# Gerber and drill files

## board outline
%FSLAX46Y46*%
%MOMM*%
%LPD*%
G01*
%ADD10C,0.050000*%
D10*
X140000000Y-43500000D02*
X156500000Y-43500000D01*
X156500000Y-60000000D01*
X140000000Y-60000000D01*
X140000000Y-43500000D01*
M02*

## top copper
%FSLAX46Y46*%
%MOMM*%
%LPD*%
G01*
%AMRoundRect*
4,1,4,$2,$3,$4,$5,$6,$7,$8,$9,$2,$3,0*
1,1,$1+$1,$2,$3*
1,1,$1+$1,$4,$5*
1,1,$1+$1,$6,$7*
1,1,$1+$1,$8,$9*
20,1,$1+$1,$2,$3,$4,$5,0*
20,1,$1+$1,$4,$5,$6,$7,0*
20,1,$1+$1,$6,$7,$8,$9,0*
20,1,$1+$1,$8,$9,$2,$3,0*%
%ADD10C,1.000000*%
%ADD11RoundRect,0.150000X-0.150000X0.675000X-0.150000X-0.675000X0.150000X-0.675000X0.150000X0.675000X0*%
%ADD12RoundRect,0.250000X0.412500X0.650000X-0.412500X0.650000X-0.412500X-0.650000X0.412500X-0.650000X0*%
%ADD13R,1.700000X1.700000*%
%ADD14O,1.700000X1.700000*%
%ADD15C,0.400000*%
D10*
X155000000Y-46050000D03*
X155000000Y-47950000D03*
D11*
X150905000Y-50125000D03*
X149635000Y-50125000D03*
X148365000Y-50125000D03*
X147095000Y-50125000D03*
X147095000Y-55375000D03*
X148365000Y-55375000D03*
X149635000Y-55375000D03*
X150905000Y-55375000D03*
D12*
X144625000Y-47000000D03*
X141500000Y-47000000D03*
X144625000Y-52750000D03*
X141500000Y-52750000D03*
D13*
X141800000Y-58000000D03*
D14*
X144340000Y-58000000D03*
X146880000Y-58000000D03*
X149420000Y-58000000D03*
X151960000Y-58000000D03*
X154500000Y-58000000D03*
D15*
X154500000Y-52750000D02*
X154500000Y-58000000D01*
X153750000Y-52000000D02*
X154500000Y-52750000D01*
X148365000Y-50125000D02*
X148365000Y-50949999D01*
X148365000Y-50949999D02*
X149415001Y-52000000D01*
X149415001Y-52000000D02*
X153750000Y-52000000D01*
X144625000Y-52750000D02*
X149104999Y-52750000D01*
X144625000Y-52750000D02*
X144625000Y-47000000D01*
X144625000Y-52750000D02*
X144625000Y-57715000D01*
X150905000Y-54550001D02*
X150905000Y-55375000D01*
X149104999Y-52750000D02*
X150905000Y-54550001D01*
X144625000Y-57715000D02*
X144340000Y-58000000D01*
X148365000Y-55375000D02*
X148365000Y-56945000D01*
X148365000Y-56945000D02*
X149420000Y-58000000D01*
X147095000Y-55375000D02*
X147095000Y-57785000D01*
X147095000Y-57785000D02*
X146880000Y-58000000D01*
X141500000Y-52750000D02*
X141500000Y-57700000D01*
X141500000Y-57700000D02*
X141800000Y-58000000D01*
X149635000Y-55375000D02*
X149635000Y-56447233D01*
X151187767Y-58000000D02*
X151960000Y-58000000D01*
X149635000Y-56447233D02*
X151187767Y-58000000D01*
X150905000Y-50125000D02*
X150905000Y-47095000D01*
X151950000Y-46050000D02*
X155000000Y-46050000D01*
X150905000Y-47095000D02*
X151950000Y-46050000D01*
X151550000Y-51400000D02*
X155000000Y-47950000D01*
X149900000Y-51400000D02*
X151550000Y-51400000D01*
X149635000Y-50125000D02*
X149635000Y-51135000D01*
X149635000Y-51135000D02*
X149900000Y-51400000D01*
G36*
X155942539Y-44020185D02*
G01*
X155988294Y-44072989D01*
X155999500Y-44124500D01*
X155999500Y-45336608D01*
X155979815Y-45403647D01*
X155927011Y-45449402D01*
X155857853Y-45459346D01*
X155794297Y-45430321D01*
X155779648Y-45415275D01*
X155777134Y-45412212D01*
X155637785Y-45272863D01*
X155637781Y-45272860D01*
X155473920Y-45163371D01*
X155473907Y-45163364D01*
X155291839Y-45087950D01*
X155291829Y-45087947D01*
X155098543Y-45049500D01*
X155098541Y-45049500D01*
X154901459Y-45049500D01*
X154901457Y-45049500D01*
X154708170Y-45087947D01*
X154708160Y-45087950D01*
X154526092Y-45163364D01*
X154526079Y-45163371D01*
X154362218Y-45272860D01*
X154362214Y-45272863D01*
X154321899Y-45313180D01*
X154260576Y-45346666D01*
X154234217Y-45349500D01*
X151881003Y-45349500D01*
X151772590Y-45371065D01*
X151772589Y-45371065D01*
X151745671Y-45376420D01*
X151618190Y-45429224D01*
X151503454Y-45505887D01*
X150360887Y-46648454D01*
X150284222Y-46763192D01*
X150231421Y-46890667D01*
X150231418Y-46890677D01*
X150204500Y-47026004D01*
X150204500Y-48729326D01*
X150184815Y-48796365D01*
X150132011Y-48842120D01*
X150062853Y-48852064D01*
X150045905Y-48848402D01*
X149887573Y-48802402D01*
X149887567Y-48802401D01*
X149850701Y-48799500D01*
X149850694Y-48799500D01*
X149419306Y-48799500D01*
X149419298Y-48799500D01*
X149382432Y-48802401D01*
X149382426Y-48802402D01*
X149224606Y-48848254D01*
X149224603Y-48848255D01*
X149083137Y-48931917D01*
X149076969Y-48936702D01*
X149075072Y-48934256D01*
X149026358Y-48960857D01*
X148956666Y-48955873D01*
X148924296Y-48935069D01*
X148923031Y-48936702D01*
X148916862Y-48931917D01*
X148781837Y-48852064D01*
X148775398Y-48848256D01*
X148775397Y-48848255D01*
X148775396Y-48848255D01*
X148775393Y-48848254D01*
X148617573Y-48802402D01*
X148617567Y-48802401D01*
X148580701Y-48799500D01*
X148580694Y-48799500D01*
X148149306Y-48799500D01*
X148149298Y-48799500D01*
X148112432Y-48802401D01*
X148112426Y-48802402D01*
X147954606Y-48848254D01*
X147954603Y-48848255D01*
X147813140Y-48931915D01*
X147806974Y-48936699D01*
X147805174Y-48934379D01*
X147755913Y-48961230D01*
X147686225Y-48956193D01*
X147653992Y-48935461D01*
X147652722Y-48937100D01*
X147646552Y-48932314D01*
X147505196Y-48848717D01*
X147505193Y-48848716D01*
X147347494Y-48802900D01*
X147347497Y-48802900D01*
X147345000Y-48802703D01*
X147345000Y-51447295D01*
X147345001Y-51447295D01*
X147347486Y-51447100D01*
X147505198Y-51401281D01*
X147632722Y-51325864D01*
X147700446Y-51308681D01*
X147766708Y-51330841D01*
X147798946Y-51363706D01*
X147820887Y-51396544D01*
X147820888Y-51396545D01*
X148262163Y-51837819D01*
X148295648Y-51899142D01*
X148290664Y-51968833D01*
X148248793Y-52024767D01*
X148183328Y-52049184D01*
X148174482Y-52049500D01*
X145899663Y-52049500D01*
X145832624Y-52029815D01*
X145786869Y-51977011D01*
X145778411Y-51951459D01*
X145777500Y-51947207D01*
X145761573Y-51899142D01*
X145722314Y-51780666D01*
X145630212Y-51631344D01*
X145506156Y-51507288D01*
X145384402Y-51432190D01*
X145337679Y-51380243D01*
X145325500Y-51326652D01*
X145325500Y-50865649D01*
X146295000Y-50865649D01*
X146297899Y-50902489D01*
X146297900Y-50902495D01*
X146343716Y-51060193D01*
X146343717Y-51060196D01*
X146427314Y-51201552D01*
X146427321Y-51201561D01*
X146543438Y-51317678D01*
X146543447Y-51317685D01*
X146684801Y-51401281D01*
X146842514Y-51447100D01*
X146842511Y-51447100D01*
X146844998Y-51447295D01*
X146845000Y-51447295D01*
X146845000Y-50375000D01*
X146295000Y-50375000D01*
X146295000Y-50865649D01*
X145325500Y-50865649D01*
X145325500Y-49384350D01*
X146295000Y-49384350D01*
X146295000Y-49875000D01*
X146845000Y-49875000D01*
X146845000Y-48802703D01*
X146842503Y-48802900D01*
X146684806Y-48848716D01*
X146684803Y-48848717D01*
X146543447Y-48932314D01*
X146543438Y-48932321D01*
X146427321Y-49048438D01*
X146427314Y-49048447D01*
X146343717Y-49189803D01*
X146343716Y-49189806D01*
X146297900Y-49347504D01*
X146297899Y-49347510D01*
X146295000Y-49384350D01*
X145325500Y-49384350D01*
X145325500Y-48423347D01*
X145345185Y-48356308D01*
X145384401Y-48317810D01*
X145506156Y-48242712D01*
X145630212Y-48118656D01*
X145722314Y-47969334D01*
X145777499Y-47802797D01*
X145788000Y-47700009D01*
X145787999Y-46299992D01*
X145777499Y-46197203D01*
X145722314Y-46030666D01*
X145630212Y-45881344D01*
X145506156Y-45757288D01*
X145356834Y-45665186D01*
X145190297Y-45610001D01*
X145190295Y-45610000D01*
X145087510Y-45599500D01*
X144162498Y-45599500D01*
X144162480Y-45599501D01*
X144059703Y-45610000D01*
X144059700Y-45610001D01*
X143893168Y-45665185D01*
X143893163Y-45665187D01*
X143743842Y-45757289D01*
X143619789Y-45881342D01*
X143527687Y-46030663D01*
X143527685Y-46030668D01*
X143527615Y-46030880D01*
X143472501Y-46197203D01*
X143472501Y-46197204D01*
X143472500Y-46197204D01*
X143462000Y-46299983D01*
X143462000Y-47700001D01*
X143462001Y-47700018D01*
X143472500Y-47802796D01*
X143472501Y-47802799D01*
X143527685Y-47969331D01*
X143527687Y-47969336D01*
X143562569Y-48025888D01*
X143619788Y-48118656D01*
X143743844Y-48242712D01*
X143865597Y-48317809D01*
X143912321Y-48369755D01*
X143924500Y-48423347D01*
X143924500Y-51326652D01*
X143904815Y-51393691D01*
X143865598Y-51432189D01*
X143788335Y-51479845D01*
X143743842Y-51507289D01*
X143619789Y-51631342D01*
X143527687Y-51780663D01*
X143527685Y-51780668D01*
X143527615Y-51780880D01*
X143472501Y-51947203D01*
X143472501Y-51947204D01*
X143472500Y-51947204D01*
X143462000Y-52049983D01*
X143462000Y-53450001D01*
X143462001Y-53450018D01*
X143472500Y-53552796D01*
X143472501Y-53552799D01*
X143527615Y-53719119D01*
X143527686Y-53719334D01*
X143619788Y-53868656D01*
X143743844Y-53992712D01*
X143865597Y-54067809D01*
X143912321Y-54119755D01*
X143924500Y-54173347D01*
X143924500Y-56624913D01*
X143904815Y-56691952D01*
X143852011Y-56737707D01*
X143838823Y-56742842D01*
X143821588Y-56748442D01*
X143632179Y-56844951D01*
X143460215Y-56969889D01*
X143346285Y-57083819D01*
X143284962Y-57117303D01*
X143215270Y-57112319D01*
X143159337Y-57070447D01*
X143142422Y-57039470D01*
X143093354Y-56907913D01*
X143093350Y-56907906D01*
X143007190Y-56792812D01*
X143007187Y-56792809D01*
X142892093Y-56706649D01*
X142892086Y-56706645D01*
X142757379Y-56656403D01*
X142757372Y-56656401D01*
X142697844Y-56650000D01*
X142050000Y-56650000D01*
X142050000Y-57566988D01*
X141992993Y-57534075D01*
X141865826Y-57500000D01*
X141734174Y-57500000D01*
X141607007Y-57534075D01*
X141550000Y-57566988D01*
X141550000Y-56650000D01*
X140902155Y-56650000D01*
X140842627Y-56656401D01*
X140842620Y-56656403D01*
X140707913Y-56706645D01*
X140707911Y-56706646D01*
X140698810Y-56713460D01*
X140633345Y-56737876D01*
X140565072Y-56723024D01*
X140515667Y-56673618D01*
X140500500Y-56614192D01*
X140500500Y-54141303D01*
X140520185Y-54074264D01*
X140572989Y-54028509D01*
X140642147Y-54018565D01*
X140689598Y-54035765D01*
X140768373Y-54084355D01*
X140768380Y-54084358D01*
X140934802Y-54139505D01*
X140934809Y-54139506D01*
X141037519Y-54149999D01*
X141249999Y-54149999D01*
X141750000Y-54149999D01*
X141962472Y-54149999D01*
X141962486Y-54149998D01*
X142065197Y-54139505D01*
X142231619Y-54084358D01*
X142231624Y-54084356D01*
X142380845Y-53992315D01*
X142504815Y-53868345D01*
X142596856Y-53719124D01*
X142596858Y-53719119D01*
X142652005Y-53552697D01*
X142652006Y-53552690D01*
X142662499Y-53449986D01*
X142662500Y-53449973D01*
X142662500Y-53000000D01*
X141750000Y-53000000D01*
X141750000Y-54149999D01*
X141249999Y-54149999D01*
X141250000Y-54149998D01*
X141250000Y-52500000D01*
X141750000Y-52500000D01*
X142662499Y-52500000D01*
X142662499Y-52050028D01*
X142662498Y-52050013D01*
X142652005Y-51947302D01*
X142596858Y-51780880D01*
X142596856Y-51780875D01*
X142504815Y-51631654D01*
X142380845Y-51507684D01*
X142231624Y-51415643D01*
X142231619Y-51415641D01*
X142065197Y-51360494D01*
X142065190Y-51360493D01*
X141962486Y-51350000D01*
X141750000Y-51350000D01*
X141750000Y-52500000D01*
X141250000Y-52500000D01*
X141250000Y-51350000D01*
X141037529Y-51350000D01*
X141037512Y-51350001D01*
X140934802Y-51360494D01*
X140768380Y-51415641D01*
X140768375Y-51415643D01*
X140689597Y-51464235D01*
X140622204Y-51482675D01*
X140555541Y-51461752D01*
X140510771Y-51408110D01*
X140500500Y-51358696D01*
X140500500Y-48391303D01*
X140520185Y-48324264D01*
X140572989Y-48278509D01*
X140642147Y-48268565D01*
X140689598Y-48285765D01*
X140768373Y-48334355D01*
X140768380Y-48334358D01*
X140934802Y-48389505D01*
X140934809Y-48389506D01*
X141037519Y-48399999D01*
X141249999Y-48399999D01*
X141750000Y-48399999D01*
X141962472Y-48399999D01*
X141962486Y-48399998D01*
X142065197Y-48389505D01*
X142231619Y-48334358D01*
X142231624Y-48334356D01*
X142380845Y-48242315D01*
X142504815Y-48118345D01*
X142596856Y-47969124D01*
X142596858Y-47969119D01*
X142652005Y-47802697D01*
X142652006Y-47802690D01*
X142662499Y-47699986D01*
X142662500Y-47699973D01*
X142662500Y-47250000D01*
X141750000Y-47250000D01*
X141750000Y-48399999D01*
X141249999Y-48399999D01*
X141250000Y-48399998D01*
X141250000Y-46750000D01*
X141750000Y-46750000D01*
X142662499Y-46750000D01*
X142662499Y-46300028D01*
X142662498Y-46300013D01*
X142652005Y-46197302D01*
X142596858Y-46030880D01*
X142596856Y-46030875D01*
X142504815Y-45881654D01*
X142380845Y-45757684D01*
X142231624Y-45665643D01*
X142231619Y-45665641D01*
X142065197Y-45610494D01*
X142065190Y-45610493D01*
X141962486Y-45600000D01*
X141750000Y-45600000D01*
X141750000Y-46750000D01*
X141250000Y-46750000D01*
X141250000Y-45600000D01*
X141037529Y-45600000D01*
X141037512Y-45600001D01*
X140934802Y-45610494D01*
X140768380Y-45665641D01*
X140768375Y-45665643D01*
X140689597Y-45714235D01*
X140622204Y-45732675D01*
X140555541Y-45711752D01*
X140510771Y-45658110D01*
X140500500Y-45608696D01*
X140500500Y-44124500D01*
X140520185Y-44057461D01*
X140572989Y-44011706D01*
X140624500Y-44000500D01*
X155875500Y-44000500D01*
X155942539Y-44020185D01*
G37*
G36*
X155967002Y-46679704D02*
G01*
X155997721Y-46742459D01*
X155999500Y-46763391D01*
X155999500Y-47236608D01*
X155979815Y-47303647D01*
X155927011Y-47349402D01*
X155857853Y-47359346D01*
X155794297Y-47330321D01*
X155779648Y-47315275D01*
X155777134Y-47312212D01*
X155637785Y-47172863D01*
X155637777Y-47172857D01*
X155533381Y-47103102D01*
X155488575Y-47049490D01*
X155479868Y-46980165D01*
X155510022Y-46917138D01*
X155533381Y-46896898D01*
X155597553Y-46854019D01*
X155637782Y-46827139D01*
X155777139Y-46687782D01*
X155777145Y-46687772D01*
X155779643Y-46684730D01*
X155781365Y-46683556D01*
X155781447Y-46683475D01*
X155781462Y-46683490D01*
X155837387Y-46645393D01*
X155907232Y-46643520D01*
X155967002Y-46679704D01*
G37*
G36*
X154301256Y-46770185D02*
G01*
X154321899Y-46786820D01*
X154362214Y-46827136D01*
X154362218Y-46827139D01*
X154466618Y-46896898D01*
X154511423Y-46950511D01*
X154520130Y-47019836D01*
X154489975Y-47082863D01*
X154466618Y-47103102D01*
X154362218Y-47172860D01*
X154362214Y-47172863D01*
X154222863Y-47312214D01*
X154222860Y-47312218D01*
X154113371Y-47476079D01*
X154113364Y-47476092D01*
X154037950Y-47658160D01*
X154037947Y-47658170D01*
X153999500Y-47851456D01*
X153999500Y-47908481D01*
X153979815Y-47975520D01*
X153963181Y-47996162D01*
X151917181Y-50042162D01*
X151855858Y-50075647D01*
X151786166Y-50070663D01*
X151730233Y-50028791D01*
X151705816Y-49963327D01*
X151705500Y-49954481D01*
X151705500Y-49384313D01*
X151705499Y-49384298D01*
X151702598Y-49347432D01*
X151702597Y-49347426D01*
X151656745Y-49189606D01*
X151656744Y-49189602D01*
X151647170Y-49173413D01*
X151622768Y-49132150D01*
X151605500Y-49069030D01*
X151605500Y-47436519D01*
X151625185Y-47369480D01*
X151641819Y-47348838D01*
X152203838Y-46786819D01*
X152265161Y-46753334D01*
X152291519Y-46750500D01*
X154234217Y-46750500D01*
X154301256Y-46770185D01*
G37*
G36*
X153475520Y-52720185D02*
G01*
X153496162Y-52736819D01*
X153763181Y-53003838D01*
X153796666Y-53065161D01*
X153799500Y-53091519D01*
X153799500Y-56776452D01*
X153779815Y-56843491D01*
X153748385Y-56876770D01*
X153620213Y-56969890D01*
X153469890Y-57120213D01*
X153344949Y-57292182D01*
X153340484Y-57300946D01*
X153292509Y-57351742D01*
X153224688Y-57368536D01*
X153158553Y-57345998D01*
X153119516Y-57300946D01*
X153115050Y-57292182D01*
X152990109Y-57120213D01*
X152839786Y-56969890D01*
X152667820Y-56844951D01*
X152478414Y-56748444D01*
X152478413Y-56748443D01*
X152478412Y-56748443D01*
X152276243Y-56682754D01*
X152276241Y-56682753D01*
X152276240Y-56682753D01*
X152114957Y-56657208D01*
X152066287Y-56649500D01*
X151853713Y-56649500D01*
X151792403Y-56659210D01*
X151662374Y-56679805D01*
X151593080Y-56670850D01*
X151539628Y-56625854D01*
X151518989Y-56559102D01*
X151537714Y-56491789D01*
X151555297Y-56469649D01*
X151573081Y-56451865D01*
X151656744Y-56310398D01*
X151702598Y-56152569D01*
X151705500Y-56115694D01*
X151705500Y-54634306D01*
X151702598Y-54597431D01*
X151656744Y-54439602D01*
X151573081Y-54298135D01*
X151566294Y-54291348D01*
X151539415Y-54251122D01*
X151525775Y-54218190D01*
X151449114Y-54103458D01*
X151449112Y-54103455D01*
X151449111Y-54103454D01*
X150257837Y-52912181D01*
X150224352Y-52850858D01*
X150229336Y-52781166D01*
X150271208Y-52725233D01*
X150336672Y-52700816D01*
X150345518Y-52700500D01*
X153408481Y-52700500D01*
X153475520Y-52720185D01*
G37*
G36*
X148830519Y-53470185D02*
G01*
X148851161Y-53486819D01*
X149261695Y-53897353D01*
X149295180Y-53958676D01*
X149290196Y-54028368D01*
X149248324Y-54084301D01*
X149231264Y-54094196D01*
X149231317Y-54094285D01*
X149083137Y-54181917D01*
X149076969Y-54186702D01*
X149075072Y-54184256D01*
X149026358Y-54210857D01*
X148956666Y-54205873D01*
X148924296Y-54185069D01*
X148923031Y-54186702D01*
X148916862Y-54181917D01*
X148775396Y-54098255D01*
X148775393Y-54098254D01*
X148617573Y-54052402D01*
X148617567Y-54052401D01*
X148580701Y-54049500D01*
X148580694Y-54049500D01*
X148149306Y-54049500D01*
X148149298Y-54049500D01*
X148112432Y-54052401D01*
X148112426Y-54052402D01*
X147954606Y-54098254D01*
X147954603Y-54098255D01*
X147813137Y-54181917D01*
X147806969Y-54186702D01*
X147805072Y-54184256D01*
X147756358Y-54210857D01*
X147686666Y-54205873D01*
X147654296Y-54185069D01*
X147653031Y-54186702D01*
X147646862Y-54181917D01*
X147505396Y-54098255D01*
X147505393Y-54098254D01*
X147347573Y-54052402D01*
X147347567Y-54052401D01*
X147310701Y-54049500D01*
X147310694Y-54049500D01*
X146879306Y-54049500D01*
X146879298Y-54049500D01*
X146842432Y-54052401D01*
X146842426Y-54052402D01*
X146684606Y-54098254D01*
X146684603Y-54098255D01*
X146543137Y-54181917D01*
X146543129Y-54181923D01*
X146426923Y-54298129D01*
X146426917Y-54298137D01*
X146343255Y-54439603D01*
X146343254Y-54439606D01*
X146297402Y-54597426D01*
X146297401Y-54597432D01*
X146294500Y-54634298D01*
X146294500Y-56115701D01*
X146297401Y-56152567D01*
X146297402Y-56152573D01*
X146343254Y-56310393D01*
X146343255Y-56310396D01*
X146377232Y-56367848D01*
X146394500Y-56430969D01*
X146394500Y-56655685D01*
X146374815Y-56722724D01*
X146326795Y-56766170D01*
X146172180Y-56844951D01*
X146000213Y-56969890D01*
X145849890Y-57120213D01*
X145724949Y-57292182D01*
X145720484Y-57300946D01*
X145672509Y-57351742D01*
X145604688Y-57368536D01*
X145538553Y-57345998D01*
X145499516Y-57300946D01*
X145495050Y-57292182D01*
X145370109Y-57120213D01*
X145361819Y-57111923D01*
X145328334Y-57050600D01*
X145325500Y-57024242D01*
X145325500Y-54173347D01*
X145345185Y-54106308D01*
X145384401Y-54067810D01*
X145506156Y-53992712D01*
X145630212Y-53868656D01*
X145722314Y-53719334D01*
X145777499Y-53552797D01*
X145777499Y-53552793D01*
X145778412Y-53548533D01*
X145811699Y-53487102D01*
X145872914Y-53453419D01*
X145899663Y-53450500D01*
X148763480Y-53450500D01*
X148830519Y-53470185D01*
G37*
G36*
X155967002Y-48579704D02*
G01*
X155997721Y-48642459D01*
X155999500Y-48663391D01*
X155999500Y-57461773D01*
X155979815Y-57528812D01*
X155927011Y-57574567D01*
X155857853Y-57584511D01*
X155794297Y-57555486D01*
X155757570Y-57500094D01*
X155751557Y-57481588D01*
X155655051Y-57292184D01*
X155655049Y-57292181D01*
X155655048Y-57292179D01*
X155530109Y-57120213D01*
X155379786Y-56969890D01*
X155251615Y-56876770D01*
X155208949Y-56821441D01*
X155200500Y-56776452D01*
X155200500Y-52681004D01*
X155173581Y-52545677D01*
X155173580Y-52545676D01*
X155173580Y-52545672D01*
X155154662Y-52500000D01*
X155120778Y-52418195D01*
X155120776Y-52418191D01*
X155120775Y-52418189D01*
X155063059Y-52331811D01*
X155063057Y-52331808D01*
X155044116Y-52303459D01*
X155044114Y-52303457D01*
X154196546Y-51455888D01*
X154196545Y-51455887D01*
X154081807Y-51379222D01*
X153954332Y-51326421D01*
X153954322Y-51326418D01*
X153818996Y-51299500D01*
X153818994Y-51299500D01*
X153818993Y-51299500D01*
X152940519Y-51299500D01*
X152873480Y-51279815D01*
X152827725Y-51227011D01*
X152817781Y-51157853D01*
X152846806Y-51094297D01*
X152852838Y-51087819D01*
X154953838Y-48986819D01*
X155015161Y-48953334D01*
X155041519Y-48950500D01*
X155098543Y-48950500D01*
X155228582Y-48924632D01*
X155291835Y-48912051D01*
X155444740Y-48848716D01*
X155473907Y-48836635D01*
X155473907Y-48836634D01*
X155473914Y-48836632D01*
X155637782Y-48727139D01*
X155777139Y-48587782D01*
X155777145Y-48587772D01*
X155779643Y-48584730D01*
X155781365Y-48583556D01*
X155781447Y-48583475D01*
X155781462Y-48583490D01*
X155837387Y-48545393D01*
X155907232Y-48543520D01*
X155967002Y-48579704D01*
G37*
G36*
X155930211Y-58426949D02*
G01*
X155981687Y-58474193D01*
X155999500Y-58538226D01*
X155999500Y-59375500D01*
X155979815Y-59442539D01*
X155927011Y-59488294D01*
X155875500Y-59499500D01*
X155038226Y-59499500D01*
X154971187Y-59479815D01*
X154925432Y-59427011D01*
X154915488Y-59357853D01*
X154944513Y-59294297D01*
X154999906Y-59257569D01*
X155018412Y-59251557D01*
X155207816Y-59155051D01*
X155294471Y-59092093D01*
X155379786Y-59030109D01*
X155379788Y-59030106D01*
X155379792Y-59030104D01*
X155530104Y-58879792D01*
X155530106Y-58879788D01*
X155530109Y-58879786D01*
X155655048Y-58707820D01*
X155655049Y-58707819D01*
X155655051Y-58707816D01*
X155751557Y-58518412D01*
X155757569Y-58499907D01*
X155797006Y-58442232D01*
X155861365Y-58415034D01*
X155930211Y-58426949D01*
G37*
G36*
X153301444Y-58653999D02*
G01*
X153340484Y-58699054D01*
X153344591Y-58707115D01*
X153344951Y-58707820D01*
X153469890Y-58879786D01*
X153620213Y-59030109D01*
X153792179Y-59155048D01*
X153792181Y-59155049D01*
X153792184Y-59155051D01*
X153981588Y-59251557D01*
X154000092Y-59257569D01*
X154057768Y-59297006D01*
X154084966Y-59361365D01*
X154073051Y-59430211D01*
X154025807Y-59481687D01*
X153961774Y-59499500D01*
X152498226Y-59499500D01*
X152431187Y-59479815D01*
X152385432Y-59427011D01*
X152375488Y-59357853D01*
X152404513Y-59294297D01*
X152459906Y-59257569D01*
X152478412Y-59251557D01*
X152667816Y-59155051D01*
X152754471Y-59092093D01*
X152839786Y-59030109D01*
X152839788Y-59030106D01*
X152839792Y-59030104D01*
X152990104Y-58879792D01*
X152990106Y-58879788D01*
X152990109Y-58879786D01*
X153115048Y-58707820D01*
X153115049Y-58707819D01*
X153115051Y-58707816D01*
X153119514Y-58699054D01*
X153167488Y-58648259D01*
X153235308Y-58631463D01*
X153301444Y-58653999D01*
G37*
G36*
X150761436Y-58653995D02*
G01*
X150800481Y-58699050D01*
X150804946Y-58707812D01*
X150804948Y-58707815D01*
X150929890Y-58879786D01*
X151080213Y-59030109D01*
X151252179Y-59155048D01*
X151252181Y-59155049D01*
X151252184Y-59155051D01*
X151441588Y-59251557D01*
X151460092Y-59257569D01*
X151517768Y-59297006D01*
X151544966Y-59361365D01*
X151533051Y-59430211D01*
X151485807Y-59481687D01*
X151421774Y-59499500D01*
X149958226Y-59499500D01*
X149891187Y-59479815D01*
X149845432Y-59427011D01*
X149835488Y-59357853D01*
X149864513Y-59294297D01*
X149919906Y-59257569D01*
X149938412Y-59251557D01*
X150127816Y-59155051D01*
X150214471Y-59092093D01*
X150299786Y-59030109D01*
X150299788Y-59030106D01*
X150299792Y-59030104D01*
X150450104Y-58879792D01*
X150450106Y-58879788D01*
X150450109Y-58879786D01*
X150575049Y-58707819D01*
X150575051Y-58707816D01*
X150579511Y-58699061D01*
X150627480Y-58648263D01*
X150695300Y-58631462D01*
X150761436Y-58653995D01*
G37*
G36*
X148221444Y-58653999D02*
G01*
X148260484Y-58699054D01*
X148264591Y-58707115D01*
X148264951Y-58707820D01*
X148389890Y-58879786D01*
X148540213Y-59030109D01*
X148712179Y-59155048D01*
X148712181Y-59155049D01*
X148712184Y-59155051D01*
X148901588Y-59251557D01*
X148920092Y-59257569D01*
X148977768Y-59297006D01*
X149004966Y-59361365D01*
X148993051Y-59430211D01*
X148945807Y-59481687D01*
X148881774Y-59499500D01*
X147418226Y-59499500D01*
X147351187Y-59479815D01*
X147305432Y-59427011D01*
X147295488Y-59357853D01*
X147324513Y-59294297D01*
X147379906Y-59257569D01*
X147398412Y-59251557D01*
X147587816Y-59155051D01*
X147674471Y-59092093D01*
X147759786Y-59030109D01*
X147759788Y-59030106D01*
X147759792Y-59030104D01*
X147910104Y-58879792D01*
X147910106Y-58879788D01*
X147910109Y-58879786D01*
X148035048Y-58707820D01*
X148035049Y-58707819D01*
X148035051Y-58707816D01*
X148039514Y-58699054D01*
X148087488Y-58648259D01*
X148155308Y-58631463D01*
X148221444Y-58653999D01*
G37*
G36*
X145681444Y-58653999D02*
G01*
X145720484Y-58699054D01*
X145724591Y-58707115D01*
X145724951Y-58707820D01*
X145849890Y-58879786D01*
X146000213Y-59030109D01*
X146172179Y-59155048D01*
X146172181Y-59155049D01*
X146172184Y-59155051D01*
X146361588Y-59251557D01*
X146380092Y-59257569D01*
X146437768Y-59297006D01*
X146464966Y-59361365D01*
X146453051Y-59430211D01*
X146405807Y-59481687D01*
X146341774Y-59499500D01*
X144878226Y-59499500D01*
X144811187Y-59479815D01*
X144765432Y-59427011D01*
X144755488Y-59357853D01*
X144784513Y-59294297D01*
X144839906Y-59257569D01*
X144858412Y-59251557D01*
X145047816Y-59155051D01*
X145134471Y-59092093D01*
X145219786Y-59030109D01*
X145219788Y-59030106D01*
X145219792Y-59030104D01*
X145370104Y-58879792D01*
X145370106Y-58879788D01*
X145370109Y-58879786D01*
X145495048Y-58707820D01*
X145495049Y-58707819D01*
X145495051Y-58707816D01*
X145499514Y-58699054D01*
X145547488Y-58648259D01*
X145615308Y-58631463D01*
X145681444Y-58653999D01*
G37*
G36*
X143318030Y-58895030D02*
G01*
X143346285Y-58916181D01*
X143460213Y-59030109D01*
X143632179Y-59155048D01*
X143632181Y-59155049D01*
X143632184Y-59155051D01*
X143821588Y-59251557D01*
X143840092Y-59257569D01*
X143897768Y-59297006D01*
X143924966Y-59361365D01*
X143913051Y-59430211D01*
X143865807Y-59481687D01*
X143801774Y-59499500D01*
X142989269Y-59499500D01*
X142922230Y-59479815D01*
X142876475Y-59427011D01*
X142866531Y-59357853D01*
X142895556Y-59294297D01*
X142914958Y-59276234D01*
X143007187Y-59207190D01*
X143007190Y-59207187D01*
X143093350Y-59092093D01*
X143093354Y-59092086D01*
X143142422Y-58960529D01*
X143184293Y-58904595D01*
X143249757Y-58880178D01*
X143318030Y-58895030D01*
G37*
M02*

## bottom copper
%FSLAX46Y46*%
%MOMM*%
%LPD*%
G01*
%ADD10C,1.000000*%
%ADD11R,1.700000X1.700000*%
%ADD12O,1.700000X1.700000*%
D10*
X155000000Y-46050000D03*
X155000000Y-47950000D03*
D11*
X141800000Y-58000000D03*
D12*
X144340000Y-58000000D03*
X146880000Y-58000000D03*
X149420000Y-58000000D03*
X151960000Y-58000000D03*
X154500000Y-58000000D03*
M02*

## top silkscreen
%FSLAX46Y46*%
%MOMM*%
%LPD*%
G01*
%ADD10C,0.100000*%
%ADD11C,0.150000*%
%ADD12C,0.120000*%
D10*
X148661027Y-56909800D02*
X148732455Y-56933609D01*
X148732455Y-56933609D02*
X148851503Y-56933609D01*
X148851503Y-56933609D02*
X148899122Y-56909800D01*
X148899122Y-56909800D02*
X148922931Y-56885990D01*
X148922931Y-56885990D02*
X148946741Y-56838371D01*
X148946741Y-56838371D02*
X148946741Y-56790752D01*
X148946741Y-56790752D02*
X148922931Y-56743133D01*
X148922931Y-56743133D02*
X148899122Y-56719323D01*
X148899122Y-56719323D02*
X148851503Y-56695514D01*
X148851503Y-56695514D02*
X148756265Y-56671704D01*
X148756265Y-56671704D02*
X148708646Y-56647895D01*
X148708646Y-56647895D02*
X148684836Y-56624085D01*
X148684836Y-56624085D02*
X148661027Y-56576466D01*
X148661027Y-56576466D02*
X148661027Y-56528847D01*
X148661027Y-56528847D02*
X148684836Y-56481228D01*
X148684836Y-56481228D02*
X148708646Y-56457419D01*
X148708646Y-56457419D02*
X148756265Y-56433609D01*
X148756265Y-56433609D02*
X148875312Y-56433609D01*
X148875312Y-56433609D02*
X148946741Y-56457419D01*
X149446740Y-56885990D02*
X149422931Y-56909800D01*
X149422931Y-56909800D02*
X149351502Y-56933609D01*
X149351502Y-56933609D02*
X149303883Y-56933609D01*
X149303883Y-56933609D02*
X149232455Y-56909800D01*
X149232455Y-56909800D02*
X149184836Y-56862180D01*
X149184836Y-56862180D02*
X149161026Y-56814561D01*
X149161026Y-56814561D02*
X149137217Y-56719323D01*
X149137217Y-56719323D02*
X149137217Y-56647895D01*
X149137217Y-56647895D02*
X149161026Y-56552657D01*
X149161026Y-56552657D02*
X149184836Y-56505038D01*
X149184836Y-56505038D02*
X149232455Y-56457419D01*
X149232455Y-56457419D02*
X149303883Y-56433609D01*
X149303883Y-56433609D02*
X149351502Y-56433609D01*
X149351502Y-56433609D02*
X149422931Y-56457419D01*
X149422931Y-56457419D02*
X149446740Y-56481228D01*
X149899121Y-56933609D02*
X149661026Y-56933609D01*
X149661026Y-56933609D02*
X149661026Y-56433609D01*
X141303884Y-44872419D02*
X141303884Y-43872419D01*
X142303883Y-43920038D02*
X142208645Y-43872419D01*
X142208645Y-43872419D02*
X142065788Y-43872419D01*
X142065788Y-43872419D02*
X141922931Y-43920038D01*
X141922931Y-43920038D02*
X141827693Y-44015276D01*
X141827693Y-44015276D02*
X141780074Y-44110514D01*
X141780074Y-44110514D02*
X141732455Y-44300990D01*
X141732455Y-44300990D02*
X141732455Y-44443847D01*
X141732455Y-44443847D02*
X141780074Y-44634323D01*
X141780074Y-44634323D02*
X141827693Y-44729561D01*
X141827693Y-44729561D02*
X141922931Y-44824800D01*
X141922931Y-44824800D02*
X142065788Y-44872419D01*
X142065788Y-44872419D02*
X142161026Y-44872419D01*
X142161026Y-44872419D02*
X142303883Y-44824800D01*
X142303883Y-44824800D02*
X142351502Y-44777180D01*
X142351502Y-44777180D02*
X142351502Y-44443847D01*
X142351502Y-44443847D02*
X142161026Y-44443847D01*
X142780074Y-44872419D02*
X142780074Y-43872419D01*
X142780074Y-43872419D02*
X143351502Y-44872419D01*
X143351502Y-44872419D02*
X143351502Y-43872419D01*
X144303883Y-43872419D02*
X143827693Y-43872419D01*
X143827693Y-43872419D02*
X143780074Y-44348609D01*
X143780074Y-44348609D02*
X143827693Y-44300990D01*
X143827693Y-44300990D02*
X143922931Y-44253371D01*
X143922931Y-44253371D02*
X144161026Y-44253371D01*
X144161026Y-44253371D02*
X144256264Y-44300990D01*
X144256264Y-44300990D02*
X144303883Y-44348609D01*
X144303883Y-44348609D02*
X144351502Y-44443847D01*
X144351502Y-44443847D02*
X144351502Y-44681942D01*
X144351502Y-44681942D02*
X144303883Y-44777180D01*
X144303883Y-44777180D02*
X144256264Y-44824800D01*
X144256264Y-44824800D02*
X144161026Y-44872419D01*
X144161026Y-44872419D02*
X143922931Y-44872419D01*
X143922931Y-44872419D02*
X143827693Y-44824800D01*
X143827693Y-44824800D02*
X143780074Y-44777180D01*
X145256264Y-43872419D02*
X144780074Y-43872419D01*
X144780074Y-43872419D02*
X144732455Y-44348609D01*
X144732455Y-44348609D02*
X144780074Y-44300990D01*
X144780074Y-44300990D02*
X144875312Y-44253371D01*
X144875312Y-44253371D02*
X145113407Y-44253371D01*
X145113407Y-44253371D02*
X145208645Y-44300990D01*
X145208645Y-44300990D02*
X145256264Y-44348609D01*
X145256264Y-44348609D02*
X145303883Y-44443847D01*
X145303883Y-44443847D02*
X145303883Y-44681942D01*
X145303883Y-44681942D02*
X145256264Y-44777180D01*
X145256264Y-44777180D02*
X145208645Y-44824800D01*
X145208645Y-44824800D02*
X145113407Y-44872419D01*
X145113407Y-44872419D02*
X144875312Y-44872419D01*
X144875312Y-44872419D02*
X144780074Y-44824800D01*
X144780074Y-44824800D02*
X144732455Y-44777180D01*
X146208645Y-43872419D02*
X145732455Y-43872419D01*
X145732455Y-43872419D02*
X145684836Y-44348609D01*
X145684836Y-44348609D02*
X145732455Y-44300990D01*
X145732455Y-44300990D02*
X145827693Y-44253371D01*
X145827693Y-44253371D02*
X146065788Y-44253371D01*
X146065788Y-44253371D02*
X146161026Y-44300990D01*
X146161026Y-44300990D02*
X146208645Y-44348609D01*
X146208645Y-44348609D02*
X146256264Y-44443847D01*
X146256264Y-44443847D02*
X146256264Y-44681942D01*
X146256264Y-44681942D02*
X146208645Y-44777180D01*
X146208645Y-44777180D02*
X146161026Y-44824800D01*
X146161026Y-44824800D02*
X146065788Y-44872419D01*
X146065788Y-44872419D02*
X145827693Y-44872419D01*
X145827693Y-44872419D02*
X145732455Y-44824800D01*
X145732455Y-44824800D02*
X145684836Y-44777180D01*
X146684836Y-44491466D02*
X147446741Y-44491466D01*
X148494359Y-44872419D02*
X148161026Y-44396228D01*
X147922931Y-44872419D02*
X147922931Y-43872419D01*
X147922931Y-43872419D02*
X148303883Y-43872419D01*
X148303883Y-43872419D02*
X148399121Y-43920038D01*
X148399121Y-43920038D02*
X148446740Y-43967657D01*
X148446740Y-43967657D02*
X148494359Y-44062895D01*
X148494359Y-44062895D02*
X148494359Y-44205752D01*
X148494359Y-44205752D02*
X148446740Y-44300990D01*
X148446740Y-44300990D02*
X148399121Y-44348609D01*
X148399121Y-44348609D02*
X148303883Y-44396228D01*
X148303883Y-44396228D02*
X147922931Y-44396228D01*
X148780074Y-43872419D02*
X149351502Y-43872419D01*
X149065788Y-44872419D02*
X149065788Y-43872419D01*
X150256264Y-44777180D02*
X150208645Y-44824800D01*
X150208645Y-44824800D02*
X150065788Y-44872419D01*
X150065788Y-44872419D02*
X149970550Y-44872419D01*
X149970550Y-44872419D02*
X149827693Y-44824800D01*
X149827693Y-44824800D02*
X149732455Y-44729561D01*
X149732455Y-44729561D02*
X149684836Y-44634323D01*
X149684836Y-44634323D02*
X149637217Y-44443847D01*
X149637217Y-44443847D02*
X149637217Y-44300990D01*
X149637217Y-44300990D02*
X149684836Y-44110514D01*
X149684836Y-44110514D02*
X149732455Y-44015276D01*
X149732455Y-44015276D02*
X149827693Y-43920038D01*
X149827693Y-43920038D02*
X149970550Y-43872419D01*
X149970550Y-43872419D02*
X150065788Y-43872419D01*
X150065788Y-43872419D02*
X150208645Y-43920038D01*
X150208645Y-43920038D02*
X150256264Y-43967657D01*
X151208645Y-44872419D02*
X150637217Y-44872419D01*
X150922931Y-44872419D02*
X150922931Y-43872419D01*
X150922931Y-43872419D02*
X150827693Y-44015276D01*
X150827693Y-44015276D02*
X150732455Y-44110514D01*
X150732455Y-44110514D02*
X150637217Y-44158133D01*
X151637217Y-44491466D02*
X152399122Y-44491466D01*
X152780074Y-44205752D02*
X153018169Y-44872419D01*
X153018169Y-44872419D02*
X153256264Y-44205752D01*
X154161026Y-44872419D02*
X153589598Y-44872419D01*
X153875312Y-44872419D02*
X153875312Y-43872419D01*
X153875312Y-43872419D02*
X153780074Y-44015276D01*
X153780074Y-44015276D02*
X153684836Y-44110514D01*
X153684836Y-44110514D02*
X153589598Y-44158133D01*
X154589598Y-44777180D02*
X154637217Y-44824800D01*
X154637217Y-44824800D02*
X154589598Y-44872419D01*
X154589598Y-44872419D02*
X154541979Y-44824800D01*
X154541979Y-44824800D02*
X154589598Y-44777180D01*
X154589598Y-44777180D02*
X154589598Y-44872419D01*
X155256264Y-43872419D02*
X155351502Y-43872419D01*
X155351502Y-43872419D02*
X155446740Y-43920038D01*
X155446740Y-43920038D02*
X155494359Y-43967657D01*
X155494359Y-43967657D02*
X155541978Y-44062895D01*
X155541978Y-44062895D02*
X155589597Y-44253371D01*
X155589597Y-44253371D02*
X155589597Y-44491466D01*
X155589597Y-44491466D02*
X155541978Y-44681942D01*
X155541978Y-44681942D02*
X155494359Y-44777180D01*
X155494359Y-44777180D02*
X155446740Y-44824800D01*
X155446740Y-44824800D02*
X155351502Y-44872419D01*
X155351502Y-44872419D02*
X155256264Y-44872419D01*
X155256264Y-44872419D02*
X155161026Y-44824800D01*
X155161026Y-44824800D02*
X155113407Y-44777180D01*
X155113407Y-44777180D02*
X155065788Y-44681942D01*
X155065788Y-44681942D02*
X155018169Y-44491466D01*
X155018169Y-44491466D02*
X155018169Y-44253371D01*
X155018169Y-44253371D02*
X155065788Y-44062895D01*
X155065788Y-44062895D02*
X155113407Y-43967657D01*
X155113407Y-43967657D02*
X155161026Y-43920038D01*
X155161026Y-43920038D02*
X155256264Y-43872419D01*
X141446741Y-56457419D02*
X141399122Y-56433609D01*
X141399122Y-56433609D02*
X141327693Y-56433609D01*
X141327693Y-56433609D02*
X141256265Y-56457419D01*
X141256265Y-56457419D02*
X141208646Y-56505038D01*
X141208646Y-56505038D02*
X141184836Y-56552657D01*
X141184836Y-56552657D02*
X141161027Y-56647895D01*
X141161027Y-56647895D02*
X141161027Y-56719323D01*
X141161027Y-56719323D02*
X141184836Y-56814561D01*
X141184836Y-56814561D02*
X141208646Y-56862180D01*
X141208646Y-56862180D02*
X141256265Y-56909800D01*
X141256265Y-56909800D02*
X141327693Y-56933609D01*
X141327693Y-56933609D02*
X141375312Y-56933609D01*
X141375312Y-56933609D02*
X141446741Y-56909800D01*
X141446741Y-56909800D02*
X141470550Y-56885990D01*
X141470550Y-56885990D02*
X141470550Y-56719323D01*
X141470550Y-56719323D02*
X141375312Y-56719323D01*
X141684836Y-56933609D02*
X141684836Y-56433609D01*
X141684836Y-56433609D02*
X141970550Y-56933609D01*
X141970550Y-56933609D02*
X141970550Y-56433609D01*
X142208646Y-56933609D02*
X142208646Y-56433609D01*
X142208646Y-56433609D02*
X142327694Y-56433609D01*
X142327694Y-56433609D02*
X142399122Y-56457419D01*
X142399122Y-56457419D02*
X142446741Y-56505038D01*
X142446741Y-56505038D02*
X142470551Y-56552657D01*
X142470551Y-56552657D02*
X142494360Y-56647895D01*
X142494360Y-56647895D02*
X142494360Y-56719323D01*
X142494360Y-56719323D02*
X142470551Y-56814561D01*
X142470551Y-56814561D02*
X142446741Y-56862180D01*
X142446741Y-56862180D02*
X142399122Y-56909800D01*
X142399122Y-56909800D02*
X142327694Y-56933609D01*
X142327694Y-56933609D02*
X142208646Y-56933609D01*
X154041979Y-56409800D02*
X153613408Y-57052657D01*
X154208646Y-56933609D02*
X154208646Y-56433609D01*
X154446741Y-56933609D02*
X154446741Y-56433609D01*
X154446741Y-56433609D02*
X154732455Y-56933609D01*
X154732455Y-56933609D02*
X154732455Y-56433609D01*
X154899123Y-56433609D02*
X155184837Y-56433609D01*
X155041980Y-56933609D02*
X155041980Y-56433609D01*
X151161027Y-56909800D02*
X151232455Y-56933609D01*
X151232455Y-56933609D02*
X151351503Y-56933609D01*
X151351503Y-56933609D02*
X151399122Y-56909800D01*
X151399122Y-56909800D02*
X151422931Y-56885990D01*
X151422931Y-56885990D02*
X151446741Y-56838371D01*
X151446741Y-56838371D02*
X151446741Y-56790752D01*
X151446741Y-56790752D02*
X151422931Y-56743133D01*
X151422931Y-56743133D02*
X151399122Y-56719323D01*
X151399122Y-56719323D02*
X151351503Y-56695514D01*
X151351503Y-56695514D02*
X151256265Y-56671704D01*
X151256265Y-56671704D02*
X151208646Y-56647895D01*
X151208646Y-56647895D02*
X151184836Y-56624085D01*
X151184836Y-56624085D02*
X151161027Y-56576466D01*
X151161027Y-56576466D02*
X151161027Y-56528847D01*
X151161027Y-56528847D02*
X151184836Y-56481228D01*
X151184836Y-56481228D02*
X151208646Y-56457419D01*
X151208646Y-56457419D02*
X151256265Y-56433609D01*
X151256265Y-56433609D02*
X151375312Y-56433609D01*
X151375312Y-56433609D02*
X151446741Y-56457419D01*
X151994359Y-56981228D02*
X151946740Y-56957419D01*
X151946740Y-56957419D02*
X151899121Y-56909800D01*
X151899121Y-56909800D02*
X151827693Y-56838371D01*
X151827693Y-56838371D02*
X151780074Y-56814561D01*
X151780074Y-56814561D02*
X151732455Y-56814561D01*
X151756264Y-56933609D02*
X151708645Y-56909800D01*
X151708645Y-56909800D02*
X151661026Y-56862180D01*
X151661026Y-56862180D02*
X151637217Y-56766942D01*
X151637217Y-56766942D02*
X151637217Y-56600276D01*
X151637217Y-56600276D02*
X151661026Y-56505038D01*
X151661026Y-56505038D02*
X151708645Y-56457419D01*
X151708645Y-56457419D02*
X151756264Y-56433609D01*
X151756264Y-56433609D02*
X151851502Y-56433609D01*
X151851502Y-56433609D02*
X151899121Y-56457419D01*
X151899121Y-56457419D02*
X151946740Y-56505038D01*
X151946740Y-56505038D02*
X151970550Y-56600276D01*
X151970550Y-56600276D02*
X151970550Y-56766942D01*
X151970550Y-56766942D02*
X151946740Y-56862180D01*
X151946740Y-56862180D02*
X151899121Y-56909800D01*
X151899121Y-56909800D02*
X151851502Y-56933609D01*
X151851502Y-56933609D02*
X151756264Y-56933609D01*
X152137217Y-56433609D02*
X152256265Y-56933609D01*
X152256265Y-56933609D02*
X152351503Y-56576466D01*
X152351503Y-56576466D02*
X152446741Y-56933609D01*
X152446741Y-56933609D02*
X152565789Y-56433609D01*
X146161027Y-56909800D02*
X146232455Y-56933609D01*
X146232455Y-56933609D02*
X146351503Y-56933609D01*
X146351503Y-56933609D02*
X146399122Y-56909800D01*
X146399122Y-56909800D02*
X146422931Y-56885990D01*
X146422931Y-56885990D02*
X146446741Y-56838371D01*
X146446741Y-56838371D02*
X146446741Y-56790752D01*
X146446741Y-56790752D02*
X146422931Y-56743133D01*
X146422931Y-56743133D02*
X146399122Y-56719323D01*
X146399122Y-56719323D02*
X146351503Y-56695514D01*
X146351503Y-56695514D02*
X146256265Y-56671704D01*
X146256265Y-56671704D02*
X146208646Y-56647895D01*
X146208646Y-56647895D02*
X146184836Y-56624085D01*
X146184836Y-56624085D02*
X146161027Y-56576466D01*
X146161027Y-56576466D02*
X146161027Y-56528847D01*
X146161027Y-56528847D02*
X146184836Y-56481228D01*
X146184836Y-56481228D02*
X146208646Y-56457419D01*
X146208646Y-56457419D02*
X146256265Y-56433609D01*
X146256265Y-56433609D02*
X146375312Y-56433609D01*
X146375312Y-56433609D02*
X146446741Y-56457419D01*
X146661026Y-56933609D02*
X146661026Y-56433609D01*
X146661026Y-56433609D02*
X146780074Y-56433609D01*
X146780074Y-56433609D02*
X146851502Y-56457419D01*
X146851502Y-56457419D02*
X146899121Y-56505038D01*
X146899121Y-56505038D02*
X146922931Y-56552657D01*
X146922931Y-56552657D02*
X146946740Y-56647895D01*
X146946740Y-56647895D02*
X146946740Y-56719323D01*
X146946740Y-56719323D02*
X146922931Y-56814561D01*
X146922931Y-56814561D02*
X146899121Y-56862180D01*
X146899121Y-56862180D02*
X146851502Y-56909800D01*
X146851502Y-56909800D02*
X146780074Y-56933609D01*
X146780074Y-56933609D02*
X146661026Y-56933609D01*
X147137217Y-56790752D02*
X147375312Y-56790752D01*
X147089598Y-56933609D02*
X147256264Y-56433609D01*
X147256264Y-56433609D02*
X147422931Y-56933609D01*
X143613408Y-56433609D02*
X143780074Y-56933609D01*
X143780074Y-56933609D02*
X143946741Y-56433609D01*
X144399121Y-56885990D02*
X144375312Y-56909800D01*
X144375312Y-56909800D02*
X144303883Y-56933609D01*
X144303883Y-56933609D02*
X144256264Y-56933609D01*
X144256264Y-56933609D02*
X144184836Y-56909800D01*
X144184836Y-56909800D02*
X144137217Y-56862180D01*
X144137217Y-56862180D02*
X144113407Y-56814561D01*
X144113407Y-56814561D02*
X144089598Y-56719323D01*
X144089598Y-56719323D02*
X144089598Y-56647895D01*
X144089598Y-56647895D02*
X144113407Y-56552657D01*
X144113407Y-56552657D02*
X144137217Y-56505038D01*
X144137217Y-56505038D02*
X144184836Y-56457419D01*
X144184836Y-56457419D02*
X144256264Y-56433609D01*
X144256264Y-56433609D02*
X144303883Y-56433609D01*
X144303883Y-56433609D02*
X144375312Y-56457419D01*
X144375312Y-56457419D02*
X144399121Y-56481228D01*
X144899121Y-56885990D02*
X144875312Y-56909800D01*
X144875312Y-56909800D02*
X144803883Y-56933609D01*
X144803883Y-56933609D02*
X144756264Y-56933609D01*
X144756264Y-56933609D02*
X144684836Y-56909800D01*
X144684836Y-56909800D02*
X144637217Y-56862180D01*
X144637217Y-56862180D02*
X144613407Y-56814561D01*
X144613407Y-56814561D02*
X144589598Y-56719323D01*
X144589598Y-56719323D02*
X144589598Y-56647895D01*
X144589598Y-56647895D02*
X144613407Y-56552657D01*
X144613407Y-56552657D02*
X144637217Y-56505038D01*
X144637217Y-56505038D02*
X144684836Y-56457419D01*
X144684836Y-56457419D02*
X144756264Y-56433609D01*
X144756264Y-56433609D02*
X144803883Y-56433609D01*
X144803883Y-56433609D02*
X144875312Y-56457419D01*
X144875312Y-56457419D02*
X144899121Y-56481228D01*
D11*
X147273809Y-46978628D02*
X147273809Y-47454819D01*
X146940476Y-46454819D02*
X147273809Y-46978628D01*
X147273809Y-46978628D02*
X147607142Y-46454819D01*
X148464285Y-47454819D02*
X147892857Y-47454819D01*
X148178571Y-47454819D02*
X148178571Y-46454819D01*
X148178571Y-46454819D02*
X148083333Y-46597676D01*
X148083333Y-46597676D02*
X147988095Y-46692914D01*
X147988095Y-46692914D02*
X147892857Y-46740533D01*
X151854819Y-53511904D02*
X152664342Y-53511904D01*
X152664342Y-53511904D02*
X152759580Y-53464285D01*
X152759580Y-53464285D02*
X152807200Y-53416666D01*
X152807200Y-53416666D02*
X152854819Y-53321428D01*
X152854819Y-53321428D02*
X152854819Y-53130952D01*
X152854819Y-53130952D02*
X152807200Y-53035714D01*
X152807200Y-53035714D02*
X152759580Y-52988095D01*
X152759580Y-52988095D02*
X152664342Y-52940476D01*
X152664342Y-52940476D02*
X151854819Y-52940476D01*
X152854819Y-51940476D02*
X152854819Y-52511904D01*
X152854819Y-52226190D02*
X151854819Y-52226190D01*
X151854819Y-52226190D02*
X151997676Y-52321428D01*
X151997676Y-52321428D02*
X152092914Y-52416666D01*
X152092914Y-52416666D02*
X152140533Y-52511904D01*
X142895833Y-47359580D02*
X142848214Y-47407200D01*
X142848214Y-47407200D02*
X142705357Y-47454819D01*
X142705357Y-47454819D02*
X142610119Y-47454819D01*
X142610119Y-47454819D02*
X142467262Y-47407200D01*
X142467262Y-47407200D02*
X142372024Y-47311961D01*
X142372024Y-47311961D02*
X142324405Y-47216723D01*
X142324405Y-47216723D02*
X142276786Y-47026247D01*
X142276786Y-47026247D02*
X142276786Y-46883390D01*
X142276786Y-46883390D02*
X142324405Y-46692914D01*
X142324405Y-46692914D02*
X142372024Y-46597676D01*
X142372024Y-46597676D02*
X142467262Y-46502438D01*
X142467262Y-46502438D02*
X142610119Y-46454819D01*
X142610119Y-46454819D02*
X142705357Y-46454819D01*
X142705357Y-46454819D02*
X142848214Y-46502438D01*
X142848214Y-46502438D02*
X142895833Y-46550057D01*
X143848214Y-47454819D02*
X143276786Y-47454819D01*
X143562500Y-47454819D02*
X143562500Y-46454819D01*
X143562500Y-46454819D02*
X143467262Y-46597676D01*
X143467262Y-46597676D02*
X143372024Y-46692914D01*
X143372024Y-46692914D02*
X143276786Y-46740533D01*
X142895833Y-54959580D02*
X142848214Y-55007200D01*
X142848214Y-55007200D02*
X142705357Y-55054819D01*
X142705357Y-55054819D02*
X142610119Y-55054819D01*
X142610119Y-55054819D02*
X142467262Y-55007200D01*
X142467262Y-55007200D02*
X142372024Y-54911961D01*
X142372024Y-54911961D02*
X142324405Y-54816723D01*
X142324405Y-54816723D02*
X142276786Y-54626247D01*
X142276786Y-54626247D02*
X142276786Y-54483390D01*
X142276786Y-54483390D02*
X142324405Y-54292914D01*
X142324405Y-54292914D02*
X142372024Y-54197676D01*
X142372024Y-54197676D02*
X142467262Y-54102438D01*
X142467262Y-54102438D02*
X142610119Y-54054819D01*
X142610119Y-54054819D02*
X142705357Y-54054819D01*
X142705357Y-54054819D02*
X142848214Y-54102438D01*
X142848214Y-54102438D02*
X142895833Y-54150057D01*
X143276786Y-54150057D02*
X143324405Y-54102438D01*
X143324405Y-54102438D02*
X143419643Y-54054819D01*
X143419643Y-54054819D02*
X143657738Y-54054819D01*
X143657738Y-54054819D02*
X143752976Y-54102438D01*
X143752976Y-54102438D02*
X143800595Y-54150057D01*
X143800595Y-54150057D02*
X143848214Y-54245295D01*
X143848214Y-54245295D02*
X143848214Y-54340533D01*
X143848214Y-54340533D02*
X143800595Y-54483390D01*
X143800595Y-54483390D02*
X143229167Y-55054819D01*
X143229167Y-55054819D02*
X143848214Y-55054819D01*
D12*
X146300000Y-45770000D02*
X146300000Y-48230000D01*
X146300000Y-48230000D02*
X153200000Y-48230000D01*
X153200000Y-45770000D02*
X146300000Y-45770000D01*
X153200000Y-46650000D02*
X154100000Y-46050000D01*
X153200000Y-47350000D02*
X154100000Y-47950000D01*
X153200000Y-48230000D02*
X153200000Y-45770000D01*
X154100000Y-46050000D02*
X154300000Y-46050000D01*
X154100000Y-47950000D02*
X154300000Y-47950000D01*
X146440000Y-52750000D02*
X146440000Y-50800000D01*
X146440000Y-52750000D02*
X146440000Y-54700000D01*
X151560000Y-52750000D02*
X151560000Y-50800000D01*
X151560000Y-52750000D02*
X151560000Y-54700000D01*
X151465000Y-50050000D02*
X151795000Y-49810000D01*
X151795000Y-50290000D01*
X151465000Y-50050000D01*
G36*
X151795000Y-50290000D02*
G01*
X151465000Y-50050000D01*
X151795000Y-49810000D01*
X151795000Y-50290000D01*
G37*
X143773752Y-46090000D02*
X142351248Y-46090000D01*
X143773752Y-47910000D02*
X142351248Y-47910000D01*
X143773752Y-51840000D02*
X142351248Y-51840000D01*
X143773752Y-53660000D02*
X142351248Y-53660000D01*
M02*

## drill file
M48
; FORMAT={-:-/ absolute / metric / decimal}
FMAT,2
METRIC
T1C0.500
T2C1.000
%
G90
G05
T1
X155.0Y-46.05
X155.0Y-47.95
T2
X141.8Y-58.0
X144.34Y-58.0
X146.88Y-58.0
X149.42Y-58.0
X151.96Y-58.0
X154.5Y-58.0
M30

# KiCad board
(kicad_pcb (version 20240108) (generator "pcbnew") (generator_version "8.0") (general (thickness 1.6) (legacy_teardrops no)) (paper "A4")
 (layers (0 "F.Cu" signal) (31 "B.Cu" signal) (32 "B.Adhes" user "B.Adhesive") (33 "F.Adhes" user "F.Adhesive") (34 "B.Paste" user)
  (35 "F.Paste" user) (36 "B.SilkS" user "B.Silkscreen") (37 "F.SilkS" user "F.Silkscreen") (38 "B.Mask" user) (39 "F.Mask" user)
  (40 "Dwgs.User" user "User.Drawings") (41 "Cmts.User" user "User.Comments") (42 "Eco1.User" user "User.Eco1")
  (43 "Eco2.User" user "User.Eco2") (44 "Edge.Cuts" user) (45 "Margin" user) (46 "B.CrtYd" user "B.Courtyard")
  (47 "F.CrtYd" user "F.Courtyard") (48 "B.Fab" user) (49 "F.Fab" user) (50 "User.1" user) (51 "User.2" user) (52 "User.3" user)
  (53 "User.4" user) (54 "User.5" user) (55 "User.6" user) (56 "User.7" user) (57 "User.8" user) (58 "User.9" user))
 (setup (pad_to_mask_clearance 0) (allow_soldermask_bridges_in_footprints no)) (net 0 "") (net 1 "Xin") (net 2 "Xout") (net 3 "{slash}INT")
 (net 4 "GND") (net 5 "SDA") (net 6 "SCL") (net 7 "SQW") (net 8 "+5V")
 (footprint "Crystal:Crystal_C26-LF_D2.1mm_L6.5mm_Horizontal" (layer "F.Cu") (at 155 46.05 -90)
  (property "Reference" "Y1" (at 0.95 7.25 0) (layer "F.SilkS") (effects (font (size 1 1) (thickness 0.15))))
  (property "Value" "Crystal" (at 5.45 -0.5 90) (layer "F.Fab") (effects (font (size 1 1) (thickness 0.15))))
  (fp_line (start -0.28 8.7) (end 2.18 8.7) (stroke (width 0.12) (type solid)) (layer "F.SilkS"))
  (fp_line (start 2.18 8.7) (end 2.18 1.8) (stroke (width 0.12) (type solid)) (layer "F.SilkS"))
  (fp_line (start -0.28 1.8) (end -0.28 8.7) (stroke (width 0.12) (type solid)) (layer "F.SilkS"))
  (fp_line (start 0.6 1.8) (end 0 0.9) (stroke (width 0.12) (type solid)) (layer "F.SilkS"))
  (fp_line (start 1.3 1.8) (end 1.9 0.9) (stroke (width 0.12) (type solid)) (layer "F.SilkS"))
  (fp_line (start 2.18 1.8) (end -0.28 1.8) (stroke (width 0.12) (type solid)) (layer "F.SilkS"))
  (fp_line (start 0 0.9) (end 0 0.7) (stroke (width 0.12) (type solid)) (layer "F.SilkS"))
  (fp_line (start 1.9 0.9) (end 1.9 0.7) (stroke (width 0.12) (type solid)) (layer "F.SilkS"))
  (pad "1" thru_hole circle (at 0 0 270) (size 1 1) (drill 0.5) (layers "*.Cu" "*.Mask") (remove_unused_layers no) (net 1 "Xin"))
  (pad "2" thru_hole circle (at 1.9 0 270) (size 1 1) (drill 0.5) (layers "*.Cu" "*.Mask") (remove_unused_layers no) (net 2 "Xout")))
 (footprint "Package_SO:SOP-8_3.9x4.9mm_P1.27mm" (layer "F.Cu") (at 149 52.75 -90)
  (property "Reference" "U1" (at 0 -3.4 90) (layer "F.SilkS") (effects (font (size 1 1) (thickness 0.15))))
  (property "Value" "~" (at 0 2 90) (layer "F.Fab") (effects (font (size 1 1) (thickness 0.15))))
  (fp_line (start 0 2.56) (end -1.95 2.56) (stroke (width 0.12) (type solid)) (layer "F.SilkS"))
  (fp_line (start 0 2.56) (end 1.95 2.56) (stroke (width 0.12) (type solid)) (layer "F.SilkS"))
  (fp_line (start 0 -2.56) (end -1.95 -2.56) (stroke (width 0.12) (type solid)) (layer "F.SilkS"))
  (fp_line (start 0 -2.56) (end 1.95 -2.56) (stroke (width 0.12) (type solid)) (layer "F.SilkS"))
  (fp_poly
   (pts (xy -2.7 -2.465) (xy -2.94 -2.795) (xy -2.46 -2.795) (xy -2.7 -2.465)) (stroke (width 0.12) (type solid)) (fill solid)
   (layer "F.SilkS"))
  (pad "1" smd roundrect (at -2.625 -1.905 270) (size 1.65 0.6) (layers "F.Cu" "F.Paste" "F.Mask") (roundrect_rratio 0.25) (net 1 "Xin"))
  (pad "2" smd roundrect (at -2.625 -0.635 270) (size 1.65 0.6) (layers "F.Cu" "F.Paste" "F.Mask") (roundrect_rratio 0.25) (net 2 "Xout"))
  (pad "3" smd roundrect (at -2.625 0.635 270) (size 1.65 0.6) (layers "F.Cu" "F.Paste" "F.Mask") (roundrect_rratio 0.25)
   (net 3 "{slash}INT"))
  (pad "4" smd roundrect (at -2.625 1.905 270) (size 1.65 0.6) (layers "F.Cu" "F.Paste" "F.Mask") (roundrect_rratio 0.25) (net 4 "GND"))
  (pad "5" smd roundrect (at 2.625 1.905 270) (size 1.65 0.6) (layers "F.Cu" "F.Paste" "F.Mask") (roundrect_rratio 0.25) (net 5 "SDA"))
  (pad "6" smd roundrect (at 2.625 0.635 270) (size 1.65 0.6) (layers "F.Cu" "F.Paste" "F.Mask") (roundrect_rratio 0.25) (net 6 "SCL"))
  (pad "7" smd roundrect (at 2.625 -0.635 270) (size 1.65 0.6) (layers "F.Cu" "F.Paste" "F.Mask") (roundrect_rratio 0.25) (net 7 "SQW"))
  (pad "8" smd roundrect (at 2.625 -1.905 270) (size 1.65 0.6) (layers "F.Cu" "F.Paste" "F.Mask") (roundrect_rratio 0.25) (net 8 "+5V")))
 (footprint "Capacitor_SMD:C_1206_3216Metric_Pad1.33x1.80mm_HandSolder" (layer "F.Cu") (at 143.0625 47 180)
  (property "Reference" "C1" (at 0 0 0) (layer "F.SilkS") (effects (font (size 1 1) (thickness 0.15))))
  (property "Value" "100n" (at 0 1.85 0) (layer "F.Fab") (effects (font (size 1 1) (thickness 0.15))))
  (fp_line (start -0.711252 0.91) (end 0.711252 0.91) (stroke (width 0.12) (type solid)) (layer "F.SilkS"))
  (fp_line (start -0.711252 -0.91) (end 0.711252 -0.91) (stroke (width 0.12) (type solid)) (layer "F.SilkS"))
  (pad "1" smd roundrect (at -1.5625 0 180) (size 1.325 1.8) (layers "F.Cu" "F.Paste" "F.Mask") (roundrect_rratio 0.188679) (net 8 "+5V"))
  (pad "2" smd roundrect (at 1.5625 0 180) (size 1.325 1.8) (layers "F.Cu" "F.Paste" "F.Mask") (roundrect_rratio 0.188679) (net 4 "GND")))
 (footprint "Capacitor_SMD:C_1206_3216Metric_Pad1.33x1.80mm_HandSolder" (layer "F.Cu") (at 143.0625 52.75 180)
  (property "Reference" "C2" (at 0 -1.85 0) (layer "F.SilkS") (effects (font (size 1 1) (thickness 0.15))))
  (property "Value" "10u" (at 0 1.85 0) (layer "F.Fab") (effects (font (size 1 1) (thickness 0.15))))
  (fp_line (start -0.711252 0.91) (end 0.711252 0.91) (stroke (width 0.12) (type solid)) (layer "F.SilkS"))
  (fp_line (start -0.711252 -0.91) (end 0.711252 -0.91) (stroke (width 0.12) (type solid)) (layer "F.SilkS"))
  (pad "1" smd roundrect (at -1.5625 0 180) (size 1.325 1.8) (layers "F.Cu" "F.Paste" "F.Mask") (roundrect_rratio 0.188679) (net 8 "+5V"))
  (pad "2" smd roundrect (at 1.5625 0 180) (size 1.325 1.8) (layers "F.Cu" "F.Paste" "F.Mask") (roundrect_rratio 0.188679) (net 4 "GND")))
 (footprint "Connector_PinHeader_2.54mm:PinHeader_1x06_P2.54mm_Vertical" (layer "B.Cu") (at 141.8 58 -90)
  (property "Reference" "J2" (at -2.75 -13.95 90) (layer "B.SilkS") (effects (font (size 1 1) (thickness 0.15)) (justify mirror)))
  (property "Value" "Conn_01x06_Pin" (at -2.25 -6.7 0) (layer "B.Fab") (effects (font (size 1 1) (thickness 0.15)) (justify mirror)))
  (pad "1" thru_hole rect (at 0 0 270) (size 1.7 1.7) (drill 1) (layers "*.Cu" "*.Mask") (remove_unused_layers no) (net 4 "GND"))
  (pad "2" thru_hole oval (at 0 -2.54 270) (size 1.7 1.7) (drill 1) (layers "*.Cu" "*.Mask") (remove_unused_layers no) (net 8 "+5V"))
  (pad "3" thru_hole oval (at 0 -5.08 270) (size 1.7 1.7) (drill 1) (layers "*.Cu" "*.Mask") (remove_unused_layers no) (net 5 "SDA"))
  (pad "4" thru_hole oval (at 0 -7.62 270) (size 1.7 1.7) (drill 1) (layers "*.Cu" "*.Mask") (remove_unused_layers no) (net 6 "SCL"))
  (pad "5" thru_hole oval (at 0 -10.16 270) (size 1.7 1.7) (drill 1) (layers "*.Cu" "*.Mask") (remove_unused_layers no) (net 7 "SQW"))
  (pad "6" thru_hole oval (at 0 -12.7 270) (size 1.7 1.7) (drill 1) (layers "*.Cu" "*.Mask") (remove_unused_layers no) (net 3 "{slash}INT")))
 (gr_rect (start 140 43.5) (end 156.5 60) (stroke (width 0.05) (type default)) (fill none) (layer "Edge.Cuts"))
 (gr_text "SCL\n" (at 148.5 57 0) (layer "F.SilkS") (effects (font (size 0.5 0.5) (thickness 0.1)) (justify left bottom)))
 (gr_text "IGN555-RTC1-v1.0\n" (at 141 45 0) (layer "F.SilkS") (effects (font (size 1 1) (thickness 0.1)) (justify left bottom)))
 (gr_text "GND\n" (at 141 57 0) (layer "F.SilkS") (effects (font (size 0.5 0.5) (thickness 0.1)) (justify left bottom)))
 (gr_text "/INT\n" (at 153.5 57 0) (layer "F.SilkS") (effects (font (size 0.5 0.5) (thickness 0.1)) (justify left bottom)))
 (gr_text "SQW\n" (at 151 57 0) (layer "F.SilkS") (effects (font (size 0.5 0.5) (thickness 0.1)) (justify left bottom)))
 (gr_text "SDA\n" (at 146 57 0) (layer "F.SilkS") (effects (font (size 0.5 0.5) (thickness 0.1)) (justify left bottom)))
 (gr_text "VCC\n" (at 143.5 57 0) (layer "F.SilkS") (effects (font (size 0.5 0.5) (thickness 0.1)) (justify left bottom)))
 (segment (start 154.5 52.75) (end 154.5 58) (width 0.4) (layer "F.Cu") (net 3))
 (segment (start 153.75 52) (end 154.5 52.75) (width 0.4) (layer "F.Cu") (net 3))
 (segment (start 148.365 50.125) (end 148.365 50.949999) (width 0.4) (layer "F.Cu") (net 3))
 (segment (start 148.365 50.949999) (end 149.415001 52) (width 0.4) (layer "F.Cu") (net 3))
 (segment (start 149.415001 52) (end 153.75 52) (width 0.4) (layer "F.Cu") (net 3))
 (segment (start 144.625 52.75) (end 149.104999 52.75) (width 0.4) (layer "F.Cu") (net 8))
 (segment (start 144.625 52.75) (end 144.625 47) (width 0.4) (layer "F.Cu") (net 8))
 (segment (start 144.625 52.75) (end 144.625 57.715) (width 0.4) (layer "F.Cu") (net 8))
 (segment (start 150.905 54.550001) (end 150.905 55.375) (width 0.4) (layer "F.Cu") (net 8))
 (segment (start 149.104999 52.75) (end 150.905 54.550001) (width 0.4) (layer "F.Cu") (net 8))
 (segment (start 144.625 57.715) (end 144.34 58) (width 0.4) (layer "F.Cu") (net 8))
 (segment (start 148.365 55.375) (end 148.365 56.945) (width 0.4) (layer "F.Cu") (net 6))
 (segment (start 148.365 56.945) (end 149.42 58) (width 0.4) (layer "F.Cu") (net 6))
 (segment (start 147.095 55.375) (end 147.095 57.785) (width 0.4) (layer "F.Cu") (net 5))
 (segment (start 147.095 57.785) (end 146.88 58) (width 0.4) (layer "F.Cu") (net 5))
 (segment (start 141.5 52.75) (end 141.5 57.7) (width 0.4) (layer "F.Cu") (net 4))
 (segment (start 141.5 57.7) (end 141.8 58) (width 0.4) (layer "F.Cu") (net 4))
 (segment (start 149.635 55.375) (end 149.635 56.447233) (width 0.4) (layer "F.Cu") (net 7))
 (segment (start 151.187767 58) (end 151.96 58) (width 0.4) (layer "F.Cu") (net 7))
 (segment (start 149.635 56.447233) (end 151.187767 58) (width 0.4) (layer "F.Cu") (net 7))
 (segment (start 150.905 50.125) (end 150.905 47.095) (width 0.4) (layer "F.Cu") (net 1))
 (segment (start 151.95 46.05) (end 155 46.05) (width 0.4) (layer "F.Cu") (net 1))
 (segment (start 150.905 47.095) (end 151.95 46.05) (width 0.4) (layer "F.Cu") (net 1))
 (segment (start 151.55 51.4) (end 155 47.95) (width 0.4) (layer "F.Cu") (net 2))
 (segment (start 149.9 51.4) (end 151.55 51.4) (width 0.4) (layer "F.Cu") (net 2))
 (segment (start 149.635 50.125) (end 149.635 51.135) (width 0.4) (layer "F.Cu") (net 2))
 (segment (start 149.635 51.135) (end 149.9 51.4) (width 0.4) (layer "F.Cu") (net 2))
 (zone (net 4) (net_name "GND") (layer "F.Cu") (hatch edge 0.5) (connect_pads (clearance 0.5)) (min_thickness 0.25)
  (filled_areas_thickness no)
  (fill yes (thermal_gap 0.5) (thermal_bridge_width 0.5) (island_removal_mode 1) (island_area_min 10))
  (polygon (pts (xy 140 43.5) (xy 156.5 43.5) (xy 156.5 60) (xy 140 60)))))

